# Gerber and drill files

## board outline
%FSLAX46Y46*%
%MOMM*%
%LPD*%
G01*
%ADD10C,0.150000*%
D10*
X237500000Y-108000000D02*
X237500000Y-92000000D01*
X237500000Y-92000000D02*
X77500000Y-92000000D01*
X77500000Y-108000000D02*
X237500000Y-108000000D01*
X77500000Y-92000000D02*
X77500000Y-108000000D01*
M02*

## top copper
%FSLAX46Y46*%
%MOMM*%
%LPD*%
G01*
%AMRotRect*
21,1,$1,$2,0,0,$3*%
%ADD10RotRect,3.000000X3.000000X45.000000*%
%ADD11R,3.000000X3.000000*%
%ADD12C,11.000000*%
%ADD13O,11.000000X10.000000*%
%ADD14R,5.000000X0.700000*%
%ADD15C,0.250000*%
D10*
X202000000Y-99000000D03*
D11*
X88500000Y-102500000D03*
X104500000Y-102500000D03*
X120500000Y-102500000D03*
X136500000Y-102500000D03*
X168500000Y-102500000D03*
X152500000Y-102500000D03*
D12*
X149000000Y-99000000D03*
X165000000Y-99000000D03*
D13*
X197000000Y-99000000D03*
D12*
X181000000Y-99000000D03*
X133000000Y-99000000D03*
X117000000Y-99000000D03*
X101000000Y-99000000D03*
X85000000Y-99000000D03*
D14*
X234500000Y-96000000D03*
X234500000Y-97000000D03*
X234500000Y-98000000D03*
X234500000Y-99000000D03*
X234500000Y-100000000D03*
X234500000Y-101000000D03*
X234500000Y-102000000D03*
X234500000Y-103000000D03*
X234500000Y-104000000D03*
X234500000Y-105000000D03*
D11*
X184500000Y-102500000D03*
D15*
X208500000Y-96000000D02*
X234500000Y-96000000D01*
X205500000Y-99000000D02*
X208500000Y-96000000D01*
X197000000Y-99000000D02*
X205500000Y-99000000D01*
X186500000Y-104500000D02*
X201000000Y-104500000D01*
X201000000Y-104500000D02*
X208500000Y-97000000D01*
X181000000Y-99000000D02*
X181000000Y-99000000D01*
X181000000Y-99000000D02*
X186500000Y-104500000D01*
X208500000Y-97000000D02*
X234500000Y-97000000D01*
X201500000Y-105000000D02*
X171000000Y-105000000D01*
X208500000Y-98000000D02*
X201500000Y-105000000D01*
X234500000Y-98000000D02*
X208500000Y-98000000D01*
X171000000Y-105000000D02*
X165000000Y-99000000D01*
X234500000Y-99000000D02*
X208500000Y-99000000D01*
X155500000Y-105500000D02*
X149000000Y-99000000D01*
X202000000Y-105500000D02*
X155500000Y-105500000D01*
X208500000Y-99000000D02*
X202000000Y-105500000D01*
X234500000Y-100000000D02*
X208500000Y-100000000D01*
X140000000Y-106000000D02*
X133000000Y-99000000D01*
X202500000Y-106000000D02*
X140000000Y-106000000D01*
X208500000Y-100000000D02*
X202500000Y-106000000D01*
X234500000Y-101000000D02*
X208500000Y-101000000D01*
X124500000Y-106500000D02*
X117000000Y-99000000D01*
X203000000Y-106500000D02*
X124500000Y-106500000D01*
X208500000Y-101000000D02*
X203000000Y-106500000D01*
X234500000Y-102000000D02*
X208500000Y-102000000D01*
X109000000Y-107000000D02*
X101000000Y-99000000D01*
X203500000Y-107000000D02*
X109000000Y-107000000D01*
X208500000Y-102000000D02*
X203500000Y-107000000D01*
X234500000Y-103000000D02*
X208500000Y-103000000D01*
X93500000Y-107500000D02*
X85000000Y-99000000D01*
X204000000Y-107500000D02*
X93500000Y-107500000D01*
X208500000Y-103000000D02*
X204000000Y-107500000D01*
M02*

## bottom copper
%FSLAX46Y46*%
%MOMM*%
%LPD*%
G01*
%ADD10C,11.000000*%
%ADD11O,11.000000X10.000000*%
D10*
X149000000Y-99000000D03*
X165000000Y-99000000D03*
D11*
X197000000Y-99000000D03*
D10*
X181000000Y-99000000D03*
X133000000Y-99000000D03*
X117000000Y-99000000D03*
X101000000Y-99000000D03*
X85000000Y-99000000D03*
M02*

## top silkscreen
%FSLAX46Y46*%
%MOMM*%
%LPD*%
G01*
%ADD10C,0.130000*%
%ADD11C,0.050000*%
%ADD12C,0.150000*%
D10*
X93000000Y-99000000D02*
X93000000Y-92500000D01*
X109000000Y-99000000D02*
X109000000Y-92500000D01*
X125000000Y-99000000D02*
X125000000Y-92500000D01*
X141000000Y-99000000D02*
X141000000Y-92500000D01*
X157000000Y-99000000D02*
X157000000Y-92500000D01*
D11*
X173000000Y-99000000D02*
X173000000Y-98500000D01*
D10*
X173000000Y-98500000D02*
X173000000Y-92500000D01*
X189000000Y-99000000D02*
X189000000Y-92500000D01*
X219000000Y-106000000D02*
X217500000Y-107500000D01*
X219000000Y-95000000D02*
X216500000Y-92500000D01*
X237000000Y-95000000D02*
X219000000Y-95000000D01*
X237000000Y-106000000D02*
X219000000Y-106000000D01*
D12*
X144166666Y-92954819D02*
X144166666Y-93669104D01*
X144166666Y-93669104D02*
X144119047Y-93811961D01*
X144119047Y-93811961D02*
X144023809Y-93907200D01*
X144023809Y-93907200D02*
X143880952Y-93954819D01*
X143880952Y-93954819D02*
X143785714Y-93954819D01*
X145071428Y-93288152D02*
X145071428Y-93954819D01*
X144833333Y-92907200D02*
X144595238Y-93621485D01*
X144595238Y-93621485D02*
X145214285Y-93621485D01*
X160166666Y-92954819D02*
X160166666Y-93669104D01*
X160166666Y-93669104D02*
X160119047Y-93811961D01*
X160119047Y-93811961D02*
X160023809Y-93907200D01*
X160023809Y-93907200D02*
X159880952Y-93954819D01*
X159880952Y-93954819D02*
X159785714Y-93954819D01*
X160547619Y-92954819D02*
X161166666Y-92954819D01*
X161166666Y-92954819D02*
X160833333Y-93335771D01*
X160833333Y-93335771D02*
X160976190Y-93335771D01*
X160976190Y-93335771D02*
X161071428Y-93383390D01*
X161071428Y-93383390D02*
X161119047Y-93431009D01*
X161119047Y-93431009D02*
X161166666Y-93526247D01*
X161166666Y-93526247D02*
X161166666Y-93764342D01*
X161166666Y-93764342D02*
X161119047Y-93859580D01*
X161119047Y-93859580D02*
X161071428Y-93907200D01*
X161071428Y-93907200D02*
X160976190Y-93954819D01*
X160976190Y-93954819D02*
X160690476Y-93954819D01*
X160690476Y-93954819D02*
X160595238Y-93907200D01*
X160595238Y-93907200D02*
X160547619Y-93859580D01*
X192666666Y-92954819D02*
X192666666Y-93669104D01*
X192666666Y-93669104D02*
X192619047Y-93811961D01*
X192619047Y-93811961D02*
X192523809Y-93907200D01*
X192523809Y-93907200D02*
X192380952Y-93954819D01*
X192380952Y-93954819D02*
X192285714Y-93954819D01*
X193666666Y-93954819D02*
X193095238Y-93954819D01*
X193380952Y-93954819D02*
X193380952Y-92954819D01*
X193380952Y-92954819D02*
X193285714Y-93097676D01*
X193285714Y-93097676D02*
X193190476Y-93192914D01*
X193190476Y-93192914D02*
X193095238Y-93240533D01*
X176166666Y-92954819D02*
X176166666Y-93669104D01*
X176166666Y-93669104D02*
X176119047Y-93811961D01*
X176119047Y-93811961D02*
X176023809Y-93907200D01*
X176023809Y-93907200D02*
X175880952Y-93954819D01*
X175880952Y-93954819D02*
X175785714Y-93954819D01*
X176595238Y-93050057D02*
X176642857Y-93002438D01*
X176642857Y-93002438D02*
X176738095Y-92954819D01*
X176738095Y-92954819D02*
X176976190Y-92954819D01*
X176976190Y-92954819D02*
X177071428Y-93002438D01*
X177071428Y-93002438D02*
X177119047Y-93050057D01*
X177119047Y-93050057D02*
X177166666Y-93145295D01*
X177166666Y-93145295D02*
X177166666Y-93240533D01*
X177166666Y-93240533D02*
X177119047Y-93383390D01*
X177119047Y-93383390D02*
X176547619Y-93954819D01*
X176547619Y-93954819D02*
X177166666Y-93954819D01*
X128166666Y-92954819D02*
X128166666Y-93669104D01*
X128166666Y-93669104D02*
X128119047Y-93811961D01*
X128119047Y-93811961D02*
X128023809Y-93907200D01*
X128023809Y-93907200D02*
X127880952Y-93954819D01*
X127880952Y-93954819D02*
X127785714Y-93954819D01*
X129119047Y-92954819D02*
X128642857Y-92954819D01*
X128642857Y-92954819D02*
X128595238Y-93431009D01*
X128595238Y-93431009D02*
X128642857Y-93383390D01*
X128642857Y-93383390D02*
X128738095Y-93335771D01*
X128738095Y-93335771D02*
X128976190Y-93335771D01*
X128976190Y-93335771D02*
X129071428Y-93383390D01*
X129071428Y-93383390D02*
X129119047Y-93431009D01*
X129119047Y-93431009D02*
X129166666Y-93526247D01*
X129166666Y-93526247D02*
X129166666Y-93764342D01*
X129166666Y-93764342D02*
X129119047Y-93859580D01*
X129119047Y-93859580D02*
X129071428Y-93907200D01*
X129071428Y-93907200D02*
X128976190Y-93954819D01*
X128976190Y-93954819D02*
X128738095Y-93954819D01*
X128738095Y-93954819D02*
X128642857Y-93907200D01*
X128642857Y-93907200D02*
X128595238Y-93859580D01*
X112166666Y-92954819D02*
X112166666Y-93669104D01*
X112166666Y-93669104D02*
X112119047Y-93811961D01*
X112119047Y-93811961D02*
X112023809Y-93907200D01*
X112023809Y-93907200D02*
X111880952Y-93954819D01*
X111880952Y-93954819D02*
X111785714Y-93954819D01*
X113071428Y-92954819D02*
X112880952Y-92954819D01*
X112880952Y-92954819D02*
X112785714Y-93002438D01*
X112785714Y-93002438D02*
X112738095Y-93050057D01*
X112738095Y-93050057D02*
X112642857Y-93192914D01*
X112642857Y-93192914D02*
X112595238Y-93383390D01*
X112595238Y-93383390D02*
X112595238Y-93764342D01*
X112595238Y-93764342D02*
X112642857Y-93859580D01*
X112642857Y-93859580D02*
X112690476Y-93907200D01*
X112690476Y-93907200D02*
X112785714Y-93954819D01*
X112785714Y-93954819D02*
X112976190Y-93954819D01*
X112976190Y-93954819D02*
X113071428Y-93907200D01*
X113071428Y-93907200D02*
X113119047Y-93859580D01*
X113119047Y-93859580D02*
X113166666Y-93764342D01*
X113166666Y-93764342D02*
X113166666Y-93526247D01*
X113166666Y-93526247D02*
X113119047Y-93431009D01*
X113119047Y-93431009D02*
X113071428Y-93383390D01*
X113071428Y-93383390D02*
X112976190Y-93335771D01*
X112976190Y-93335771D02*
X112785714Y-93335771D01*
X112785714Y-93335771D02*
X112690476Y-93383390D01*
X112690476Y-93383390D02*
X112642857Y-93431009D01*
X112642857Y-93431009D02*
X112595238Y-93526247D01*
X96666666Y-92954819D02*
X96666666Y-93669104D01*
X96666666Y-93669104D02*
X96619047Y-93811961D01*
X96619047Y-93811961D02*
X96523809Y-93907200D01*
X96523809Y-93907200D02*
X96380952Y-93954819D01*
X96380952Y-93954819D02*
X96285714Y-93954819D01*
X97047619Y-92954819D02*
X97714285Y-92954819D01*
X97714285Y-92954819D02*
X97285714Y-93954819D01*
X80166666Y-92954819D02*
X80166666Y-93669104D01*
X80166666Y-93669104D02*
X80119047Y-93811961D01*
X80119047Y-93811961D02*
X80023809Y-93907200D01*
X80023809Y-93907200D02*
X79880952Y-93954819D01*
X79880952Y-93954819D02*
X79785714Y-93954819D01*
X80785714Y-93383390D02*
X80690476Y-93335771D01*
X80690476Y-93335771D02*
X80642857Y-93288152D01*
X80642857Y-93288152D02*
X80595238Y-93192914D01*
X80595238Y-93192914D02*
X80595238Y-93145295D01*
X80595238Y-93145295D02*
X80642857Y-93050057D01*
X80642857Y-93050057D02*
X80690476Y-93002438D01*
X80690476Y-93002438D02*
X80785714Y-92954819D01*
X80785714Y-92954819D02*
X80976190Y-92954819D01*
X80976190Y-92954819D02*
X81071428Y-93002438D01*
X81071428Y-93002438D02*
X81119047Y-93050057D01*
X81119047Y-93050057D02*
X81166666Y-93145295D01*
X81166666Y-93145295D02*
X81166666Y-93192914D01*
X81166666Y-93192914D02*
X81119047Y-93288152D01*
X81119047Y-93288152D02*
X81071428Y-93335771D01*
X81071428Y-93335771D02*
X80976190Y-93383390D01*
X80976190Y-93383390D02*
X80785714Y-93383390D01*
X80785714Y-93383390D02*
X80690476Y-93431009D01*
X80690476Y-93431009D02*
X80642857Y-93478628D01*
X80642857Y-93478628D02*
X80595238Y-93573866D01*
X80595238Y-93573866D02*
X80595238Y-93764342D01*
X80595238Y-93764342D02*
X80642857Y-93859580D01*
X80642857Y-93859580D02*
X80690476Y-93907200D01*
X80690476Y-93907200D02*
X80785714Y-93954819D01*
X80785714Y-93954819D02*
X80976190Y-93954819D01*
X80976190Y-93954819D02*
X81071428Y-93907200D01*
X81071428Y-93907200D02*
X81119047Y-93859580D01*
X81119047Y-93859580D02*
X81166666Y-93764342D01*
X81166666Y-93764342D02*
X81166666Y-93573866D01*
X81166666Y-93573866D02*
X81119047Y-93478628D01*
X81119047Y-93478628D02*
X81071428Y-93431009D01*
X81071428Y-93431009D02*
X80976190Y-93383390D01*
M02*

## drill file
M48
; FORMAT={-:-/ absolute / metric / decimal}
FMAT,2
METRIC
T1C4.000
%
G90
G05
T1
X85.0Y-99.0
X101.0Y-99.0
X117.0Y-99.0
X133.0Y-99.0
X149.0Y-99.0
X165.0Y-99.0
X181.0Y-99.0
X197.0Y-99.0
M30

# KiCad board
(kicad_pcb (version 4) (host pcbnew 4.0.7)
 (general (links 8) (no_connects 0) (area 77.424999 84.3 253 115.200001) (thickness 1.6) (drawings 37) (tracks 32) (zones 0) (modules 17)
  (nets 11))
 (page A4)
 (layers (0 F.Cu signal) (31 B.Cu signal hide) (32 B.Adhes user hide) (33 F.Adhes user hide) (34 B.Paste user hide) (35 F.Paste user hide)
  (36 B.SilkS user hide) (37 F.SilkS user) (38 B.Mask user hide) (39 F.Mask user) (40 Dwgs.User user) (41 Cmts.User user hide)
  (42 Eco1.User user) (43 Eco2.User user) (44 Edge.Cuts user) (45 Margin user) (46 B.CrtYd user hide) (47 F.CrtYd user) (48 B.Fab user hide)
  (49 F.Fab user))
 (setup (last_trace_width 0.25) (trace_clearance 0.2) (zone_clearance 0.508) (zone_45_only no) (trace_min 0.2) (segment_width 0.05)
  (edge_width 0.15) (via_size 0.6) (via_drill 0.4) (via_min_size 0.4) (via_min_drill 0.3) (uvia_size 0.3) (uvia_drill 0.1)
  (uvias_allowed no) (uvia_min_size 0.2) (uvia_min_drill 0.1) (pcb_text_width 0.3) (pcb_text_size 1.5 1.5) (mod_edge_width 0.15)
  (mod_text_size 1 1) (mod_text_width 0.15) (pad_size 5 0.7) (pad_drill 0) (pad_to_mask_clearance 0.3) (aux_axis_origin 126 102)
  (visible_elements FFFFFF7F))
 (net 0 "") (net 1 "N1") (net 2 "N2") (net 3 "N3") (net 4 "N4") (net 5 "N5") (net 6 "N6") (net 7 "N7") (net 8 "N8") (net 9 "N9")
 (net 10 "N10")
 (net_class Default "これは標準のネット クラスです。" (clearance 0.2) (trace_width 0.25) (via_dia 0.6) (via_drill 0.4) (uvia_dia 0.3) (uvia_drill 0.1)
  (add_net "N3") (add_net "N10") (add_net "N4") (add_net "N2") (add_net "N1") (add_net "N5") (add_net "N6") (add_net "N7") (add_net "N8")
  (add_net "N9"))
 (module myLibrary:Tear (layer F.Cu) (at 202 98.5)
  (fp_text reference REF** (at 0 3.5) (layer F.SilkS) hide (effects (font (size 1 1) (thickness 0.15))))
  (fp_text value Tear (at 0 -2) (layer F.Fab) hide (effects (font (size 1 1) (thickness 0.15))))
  (pad "" connect rect (at 0 0.5 45) (size 3 3) (layers F.Cu F.Mask)))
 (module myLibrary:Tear (layer F.Cu) (at 88.5 102)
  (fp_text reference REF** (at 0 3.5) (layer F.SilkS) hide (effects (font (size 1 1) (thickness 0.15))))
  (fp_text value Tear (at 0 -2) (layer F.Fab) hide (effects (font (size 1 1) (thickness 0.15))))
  (pad "" connect rect (at 0 0.5) (size 3 3) (layers F.Cu F.Mask)))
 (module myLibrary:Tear (layer F.Cu) (at 104.5 102)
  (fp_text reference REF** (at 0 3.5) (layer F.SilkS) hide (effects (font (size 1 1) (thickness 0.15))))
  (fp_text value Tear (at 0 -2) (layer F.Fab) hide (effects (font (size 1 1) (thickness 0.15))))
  (pad "" connect rect (at 0 0.5) (size 3 3) (layers F.Cu F.Mask)))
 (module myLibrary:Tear (layer F.Cu) (at 120.5 102)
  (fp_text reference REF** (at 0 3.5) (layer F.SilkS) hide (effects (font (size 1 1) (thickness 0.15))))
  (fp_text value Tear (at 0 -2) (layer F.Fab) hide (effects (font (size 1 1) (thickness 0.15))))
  (pad "" connect rect (at 0 0.5) (size 3 3) (layers F.Cu F.Mask)))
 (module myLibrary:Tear (layer F.Cu) (at 136.5 102)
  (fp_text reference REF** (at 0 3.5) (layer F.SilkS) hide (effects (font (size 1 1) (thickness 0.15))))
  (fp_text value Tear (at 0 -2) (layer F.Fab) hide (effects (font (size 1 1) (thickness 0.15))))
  (pad "" connect rect (at 0 0.5) (size 3 3) (layers F.Cu F.Mask)))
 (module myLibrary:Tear (layer F.Cu) (at 168.5 102)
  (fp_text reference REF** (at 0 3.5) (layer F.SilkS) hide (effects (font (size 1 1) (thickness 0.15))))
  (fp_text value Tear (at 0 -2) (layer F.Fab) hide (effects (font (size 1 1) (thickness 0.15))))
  (pad "" connect rect (at 0 0.5) (size 3 3) (layers F.Cu F.Mask)))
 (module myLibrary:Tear (layer F.Cu) (at 152.5 102)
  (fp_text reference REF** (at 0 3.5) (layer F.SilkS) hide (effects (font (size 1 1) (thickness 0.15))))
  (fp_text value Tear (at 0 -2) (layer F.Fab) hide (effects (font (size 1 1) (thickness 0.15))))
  (pad "" connect rect (at 0 0.5) (size 3 3) (layers F.Cu F.Mask)))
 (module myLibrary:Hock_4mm (layer F.Cu) (at 149 99)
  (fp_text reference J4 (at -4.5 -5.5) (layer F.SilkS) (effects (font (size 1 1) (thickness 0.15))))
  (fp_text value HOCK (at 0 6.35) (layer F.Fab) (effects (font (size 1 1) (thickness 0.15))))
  (pad 4 thru_hole circle (at 0 0) (size 11 11) (drill 4) (layers *.Cu *.Mask) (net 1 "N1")))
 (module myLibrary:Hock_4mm (layer F.Cu) (at 165 99)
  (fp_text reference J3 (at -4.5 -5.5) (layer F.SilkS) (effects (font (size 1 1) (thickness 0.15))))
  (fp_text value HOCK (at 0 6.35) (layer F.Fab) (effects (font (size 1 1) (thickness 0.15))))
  (pad 3 thru_hole circle (at 0 0) (size 11 11) (drill 4) (layers *.Cu *.Mask) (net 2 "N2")))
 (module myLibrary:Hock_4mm (layer F.Cu) (at 197 99)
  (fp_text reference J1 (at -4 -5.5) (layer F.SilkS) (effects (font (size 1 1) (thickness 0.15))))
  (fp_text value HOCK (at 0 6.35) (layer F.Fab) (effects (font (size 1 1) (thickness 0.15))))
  (pad 1 thru_hole oval (at 0 0) (size 11 10) (drill 4) (layers *.Cu *.Mask) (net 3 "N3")))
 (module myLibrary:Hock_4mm (layer F.Cu) (at 181 99)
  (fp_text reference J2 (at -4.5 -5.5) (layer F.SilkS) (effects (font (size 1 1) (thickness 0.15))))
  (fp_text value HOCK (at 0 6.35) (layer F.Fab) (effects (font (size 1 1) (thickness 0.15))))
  (pad 2 thru_hole circle (at 0 0) (size 11 11) (drill 4) (layers *.Cu *.Mask) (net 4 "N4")))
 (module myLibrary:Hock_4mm (layer F.Cu) (at 133 99)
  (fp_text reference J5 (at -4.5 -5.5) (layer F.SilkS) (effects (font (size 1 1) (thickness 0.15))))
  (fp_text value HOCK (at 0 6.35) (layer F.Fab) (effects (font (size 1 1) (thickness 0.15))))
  (pad 5 thru_hole circle (at 0 0) (size 11 11) (drill 4) (layers *.Cu *.Mask) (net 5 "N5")))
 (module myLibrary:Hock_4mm (layer F.Cu) (at 117 99)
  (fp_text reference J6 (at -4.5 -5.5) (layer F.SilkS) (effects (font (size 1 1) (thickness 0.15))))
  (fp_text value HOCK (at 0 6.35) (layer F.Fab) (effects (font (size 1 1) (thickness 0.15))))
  (pad 6 thru_hole circle (at 0 0) (size 11 11) (drill 4) (layers *.Cu *.Mask) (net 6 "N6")))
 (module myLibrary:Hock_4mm (layer F.Cu) (at 101 99)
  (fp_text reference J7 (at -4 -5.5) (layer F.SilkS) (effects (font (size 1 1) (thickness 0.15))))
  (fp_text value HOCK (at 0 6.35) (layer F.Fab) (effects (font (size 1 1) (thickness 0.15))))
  (pad 7 thru_hole circle (at 0 0) (size 11 11) (drill 4) (layers *.Cu *.Mask) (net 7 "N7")))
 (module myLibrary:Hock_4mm (layer F.Cu) (at 85 99)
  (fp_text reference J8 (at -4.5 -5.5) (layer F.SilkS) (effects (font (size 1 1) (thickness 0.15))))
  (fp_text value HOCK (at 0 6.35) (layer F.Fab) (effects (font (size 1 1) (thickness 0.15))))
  (pad 8 thru_hole circle (at 0 0) (size 11 11) (drill 4) (layers *.Cu *.Mask) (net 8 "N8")))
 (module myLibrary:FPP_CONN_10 (layer F.Cu) (at 234.5 100)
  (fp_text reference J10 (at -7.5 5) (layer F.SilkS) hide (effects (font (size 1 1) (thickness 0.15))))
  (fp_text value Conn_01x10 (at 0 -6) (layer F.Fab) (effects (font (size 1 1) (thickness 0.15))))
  (pad 1 smd rect (at 0 -4) (size 5 0.7) (layers F.Cu F.Paste) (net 3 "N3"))
  (pad 2 smd rect (at 0 -3) (size 5 0.7) (layers F.Cu F.Paste) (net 4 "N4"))
  (pad 3 smd rect (at 0 -2) (size 5 0.7) (layers F.Cu F.Paste) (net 2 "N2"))
  (pad 4 smd rect (at 0 -1) (size 5 0.7) (layers F.Cu F.Paste) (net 1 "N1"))
  (pad 5 smd rect (at 0 0) (size 5 0.7) (layers F.Cu F.Paste) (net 5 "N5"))
  (pad 6 smd rect (at 0 1) (size 5 0.7) (layers F.Cu F.Paste) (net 6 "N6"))
  (pad 7 smd rect (at 0 2) (size 5 0.7) (layers F.Cu F.Paste) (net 7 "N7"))
  (pad 8 smd rect (at 0 3) (size 5 0.7) (layers F.Cu F.Paste) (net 8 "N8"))
  (pad 9 smd rect (at 0 4) (size 5 0.7) (layers F.Cu F.Paste) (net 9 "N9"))
  (pad 10 smd rect (at 0 5) (size 5 0.7) (layers F.Cu F.Paste) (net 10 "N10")))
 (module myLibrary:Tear (layer F.Cu) (at 184.5 102)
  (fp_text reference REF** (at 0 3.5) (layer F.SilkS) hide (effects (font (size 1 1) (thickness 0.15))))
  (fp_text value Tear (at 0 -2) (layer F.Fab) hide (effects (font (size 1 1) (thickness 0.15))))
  (pad "" connect rect (at 0 0.5) (size 3 3) (layers F.Cu F.Mask)))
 (gr_line (start 93 99) (end 93 92.5) (angle 90) (layer F.SilkS) (width 0.13))
 (gr_line (start 109 99) (end 109 92.5) (angle 90) (layer F.SilkS) (width 0.13))
 (gr_line (start 125 99) (end 125 92.5) (angle 90) (layer F.SilkS) (width 0.13))
 (gr_line (start 141 99) (end 141 92.5) (angle 90) (layer F.SilkS) (width 0.13))
 (gr_line (start 157 99) (end 157 92.5) (angle 90) (layer F.SilkS) (width 0.13))
 (gr_line (start 173 99) (end 173 98.5) (angle 90) (layer F.SilkS) (width 0.05))
 (gr_line (start 173 98.5) (end 173 92.5) (angle 90) (layer F.SilkS) (width 0.13))
 (gr_line (start 189 99) (end 189 92.5) (angle 90) (layer F.SilkS) (width 0.13))
 (gr_line (start 219 106) (end 217.5 107.5) (angle 90) (layer F.SilkS) (width 0.13))
 (gr_line (start 219 95) (end 216.5 92.5) (angle 90) (layer F.SilkS) (width 0.13))
 (gr_line (start 237 95) (end 219 95) (angle 90) (layer F.SilkS) (width 0.13))
 (gr_line (start 237 106) (end 219 106) (angle 90) (layer F.SilkS) (width 0.13))
 (gr_line (start 237.5 108) (end 237.5 92) (angle 90) (layer Edge.Cuts) (width 0.15))
 (gr_line (start 237.5 92) (end 77.5 92) (angle 90) (layer Edge.Cuts) (width 0.15))
 (gr_line (start 77.5 108) (end 237.5 108) (angle 90) (layer Edge.Cuts) (width 0.15))
 (gr_line (start 77.5 92) (end 77.5 108) (angle 90) (layer Edge.Cuts) (width 0.15))
 (segment (start 208.5 96) (end 234.5 96) (width 0.25) (layer F.Cu) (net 3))
 (segment (start 205.5 99) (end 208.5 96) (width 0.25) (layer F.Cu) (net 3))
 (segment (start 197 99) (end 205.5 99) (width 0.25) (layer F.Cu) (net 3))
 (segment (start 186.5 104.5) (end 201 104.5) (width 0.25) (layer F.Cu) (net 4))
 (segment (start 201 104.5) (end 208.5 97) (width 0.25) (layer F.Cu) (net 4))
 (segment (start 181 99) (end 181 99) (width 0.25) (layer F.Cu) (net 4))
 (segment (start 181 99) (end 186.5 104.5) (width 0.25) (layer F.Cu) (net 4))
 (segment (start 208.5 97) (end 234.5 97) (width 0.25) (layer F.Cu) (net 4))
 (segment (start 201.5 105) (end 171 105) (width 0.25) (layer F.Cu) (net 2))
 (segment (start 208.5 98) (end 201.5 105) (width 0.25) (layer F.Cu) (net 2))
 (segment (start 234.5 98) (end 208.5 98) (width 0.25) (layer F.Cu) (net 2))
 (segment (start 171 105) (end 165 99) (width 0.25) (layer F.Cu) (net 2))
 (segment (start 234.5 99) (end 208.5 99) (width 0.25) (layer F.Cu) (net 1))
 (segment (start 155.5 105.5) (end 149 99) (width 0.25) (layer F.Cu) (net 1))
 (segment (start 202 105.5) (end 155.5 105.5) (width 0.25) (layer F.Cu) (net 1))
 (segment (start 208.5 99) (end 202 105.5) (width 0.25) (layer F.Cu) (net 1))
 (segment (start 234.5 100) (end 208.5 100) (width 0.25) (layer F.Cu) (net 5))
 (segment (start 140 106) (end 133 99) (width 0.25) (layer F.Cu) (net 5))
 (segment (start 202.5 106) (end 140 106) (width 0.25) (layer F.Cu) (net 5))
 (segment (start 208.5 100) (end 202.5 106) (width 0.25) (layer F.Cu) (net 5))
 (segment (start 234.5 101) (end 208.5 101) (width 0.25) (layer F.Cu) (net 6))
 (segment (start 124.5 106.5) (end 117 99) (width 0.25) (layer F.Cu) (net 6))
 (segment (start 203 106.5) (end 124.5 106.5) (width 0.25) (layer F.Cu) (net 6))
 (segment (start 208.5 101) (end 203 106.5) (width 0.25) (layer F.Cu) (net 6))
 (segment (start 234.5 102) (end 208.5 102) (width 0.25) (layer F.Cu) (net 7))
 (segment (start 109 107) (end 101 99) (width 0.25) (layer F.Cu) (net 7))
 (segment (start 203.5 107) (end 109 107) (width 0.25) (layer F.Cu) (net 7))
 (segment (start 208.5 102) (end 203.5 107) (width 0.25) (layer F.Cu) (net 7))
 (segment (start 234.5 103) (end 208.5 103) (width 0.25) (layer F.Cu) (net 8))
 (segment (start 93.5 107.5) (end 85 99) (width 0.25) (layer F.Cu) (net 8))
 (segment (start 204 107.5) (end 93.5 107.5) (width 0.25) (layer F.Cu) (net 8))
 (segment (start 208.5 103) (end 204 107.5) (width 0.25) (layer F.Cu) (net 8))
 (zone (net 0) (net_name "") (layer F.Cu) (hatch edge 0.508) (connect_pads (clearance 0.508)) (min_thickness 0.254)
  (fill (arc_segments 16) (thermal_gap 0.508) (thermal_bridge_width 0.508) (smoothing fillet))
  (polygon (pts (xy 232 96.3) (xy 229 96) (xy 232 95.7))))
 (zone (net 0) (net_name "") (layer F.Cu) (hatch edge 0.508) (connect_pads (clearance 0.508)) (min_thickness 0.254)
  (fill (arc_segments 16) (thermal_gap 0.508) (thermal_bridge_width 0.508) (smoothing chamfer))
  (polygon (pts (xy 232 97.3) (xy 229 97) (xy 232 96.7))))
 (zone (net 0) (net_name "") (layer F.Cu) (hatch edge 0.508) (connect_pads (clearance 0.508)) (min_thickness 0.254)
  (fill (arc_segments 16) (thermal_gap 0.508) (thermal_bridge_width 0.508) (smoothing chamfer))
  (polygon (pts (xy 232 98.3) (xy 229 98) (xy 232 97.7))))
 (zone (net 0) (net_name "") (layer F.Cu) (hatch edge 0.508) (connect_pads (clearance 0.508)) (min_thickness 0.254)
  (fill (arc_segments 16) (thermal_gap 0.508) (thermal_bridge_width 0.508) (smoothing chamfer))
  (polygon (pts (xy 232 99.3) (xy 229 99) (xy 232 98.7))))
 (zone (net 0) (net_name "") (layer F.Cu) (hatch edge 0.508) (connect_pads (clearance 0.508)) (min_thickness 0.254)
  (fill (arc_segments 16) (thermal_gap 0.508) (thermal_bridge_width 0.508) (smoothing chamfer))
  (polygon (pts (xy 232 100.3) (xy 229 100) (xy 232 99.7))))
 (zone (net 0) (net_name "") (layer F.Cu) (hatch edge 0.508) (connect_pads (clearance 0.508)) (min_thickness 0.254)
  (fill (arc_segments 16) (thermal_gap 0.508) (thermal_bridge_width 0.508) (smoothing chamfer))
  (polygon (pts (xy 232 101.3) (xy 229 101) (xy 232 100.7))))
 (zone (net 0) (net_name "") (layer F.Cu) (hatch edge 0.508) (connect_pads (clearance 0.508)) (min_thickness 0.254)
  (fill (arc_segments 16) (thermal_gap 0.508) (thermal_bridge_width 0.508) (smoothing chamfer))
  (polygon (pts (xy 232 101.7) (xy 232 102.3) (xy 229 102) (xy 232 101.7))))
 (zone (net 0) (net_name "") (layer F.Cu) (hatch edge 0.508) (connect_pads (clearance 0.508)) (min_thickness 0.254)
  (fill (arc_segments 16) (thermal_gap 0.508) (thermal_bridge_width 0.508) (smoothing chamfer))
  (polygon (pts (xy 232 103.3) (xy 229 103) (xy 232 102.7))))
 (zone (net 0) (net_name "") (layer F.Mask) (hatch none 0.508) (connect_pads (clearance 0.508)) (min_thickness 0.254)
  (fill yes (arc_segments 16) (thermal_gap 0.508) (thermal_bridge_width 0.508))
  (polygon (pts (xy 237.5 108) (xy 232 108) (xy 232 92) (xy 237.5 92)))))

